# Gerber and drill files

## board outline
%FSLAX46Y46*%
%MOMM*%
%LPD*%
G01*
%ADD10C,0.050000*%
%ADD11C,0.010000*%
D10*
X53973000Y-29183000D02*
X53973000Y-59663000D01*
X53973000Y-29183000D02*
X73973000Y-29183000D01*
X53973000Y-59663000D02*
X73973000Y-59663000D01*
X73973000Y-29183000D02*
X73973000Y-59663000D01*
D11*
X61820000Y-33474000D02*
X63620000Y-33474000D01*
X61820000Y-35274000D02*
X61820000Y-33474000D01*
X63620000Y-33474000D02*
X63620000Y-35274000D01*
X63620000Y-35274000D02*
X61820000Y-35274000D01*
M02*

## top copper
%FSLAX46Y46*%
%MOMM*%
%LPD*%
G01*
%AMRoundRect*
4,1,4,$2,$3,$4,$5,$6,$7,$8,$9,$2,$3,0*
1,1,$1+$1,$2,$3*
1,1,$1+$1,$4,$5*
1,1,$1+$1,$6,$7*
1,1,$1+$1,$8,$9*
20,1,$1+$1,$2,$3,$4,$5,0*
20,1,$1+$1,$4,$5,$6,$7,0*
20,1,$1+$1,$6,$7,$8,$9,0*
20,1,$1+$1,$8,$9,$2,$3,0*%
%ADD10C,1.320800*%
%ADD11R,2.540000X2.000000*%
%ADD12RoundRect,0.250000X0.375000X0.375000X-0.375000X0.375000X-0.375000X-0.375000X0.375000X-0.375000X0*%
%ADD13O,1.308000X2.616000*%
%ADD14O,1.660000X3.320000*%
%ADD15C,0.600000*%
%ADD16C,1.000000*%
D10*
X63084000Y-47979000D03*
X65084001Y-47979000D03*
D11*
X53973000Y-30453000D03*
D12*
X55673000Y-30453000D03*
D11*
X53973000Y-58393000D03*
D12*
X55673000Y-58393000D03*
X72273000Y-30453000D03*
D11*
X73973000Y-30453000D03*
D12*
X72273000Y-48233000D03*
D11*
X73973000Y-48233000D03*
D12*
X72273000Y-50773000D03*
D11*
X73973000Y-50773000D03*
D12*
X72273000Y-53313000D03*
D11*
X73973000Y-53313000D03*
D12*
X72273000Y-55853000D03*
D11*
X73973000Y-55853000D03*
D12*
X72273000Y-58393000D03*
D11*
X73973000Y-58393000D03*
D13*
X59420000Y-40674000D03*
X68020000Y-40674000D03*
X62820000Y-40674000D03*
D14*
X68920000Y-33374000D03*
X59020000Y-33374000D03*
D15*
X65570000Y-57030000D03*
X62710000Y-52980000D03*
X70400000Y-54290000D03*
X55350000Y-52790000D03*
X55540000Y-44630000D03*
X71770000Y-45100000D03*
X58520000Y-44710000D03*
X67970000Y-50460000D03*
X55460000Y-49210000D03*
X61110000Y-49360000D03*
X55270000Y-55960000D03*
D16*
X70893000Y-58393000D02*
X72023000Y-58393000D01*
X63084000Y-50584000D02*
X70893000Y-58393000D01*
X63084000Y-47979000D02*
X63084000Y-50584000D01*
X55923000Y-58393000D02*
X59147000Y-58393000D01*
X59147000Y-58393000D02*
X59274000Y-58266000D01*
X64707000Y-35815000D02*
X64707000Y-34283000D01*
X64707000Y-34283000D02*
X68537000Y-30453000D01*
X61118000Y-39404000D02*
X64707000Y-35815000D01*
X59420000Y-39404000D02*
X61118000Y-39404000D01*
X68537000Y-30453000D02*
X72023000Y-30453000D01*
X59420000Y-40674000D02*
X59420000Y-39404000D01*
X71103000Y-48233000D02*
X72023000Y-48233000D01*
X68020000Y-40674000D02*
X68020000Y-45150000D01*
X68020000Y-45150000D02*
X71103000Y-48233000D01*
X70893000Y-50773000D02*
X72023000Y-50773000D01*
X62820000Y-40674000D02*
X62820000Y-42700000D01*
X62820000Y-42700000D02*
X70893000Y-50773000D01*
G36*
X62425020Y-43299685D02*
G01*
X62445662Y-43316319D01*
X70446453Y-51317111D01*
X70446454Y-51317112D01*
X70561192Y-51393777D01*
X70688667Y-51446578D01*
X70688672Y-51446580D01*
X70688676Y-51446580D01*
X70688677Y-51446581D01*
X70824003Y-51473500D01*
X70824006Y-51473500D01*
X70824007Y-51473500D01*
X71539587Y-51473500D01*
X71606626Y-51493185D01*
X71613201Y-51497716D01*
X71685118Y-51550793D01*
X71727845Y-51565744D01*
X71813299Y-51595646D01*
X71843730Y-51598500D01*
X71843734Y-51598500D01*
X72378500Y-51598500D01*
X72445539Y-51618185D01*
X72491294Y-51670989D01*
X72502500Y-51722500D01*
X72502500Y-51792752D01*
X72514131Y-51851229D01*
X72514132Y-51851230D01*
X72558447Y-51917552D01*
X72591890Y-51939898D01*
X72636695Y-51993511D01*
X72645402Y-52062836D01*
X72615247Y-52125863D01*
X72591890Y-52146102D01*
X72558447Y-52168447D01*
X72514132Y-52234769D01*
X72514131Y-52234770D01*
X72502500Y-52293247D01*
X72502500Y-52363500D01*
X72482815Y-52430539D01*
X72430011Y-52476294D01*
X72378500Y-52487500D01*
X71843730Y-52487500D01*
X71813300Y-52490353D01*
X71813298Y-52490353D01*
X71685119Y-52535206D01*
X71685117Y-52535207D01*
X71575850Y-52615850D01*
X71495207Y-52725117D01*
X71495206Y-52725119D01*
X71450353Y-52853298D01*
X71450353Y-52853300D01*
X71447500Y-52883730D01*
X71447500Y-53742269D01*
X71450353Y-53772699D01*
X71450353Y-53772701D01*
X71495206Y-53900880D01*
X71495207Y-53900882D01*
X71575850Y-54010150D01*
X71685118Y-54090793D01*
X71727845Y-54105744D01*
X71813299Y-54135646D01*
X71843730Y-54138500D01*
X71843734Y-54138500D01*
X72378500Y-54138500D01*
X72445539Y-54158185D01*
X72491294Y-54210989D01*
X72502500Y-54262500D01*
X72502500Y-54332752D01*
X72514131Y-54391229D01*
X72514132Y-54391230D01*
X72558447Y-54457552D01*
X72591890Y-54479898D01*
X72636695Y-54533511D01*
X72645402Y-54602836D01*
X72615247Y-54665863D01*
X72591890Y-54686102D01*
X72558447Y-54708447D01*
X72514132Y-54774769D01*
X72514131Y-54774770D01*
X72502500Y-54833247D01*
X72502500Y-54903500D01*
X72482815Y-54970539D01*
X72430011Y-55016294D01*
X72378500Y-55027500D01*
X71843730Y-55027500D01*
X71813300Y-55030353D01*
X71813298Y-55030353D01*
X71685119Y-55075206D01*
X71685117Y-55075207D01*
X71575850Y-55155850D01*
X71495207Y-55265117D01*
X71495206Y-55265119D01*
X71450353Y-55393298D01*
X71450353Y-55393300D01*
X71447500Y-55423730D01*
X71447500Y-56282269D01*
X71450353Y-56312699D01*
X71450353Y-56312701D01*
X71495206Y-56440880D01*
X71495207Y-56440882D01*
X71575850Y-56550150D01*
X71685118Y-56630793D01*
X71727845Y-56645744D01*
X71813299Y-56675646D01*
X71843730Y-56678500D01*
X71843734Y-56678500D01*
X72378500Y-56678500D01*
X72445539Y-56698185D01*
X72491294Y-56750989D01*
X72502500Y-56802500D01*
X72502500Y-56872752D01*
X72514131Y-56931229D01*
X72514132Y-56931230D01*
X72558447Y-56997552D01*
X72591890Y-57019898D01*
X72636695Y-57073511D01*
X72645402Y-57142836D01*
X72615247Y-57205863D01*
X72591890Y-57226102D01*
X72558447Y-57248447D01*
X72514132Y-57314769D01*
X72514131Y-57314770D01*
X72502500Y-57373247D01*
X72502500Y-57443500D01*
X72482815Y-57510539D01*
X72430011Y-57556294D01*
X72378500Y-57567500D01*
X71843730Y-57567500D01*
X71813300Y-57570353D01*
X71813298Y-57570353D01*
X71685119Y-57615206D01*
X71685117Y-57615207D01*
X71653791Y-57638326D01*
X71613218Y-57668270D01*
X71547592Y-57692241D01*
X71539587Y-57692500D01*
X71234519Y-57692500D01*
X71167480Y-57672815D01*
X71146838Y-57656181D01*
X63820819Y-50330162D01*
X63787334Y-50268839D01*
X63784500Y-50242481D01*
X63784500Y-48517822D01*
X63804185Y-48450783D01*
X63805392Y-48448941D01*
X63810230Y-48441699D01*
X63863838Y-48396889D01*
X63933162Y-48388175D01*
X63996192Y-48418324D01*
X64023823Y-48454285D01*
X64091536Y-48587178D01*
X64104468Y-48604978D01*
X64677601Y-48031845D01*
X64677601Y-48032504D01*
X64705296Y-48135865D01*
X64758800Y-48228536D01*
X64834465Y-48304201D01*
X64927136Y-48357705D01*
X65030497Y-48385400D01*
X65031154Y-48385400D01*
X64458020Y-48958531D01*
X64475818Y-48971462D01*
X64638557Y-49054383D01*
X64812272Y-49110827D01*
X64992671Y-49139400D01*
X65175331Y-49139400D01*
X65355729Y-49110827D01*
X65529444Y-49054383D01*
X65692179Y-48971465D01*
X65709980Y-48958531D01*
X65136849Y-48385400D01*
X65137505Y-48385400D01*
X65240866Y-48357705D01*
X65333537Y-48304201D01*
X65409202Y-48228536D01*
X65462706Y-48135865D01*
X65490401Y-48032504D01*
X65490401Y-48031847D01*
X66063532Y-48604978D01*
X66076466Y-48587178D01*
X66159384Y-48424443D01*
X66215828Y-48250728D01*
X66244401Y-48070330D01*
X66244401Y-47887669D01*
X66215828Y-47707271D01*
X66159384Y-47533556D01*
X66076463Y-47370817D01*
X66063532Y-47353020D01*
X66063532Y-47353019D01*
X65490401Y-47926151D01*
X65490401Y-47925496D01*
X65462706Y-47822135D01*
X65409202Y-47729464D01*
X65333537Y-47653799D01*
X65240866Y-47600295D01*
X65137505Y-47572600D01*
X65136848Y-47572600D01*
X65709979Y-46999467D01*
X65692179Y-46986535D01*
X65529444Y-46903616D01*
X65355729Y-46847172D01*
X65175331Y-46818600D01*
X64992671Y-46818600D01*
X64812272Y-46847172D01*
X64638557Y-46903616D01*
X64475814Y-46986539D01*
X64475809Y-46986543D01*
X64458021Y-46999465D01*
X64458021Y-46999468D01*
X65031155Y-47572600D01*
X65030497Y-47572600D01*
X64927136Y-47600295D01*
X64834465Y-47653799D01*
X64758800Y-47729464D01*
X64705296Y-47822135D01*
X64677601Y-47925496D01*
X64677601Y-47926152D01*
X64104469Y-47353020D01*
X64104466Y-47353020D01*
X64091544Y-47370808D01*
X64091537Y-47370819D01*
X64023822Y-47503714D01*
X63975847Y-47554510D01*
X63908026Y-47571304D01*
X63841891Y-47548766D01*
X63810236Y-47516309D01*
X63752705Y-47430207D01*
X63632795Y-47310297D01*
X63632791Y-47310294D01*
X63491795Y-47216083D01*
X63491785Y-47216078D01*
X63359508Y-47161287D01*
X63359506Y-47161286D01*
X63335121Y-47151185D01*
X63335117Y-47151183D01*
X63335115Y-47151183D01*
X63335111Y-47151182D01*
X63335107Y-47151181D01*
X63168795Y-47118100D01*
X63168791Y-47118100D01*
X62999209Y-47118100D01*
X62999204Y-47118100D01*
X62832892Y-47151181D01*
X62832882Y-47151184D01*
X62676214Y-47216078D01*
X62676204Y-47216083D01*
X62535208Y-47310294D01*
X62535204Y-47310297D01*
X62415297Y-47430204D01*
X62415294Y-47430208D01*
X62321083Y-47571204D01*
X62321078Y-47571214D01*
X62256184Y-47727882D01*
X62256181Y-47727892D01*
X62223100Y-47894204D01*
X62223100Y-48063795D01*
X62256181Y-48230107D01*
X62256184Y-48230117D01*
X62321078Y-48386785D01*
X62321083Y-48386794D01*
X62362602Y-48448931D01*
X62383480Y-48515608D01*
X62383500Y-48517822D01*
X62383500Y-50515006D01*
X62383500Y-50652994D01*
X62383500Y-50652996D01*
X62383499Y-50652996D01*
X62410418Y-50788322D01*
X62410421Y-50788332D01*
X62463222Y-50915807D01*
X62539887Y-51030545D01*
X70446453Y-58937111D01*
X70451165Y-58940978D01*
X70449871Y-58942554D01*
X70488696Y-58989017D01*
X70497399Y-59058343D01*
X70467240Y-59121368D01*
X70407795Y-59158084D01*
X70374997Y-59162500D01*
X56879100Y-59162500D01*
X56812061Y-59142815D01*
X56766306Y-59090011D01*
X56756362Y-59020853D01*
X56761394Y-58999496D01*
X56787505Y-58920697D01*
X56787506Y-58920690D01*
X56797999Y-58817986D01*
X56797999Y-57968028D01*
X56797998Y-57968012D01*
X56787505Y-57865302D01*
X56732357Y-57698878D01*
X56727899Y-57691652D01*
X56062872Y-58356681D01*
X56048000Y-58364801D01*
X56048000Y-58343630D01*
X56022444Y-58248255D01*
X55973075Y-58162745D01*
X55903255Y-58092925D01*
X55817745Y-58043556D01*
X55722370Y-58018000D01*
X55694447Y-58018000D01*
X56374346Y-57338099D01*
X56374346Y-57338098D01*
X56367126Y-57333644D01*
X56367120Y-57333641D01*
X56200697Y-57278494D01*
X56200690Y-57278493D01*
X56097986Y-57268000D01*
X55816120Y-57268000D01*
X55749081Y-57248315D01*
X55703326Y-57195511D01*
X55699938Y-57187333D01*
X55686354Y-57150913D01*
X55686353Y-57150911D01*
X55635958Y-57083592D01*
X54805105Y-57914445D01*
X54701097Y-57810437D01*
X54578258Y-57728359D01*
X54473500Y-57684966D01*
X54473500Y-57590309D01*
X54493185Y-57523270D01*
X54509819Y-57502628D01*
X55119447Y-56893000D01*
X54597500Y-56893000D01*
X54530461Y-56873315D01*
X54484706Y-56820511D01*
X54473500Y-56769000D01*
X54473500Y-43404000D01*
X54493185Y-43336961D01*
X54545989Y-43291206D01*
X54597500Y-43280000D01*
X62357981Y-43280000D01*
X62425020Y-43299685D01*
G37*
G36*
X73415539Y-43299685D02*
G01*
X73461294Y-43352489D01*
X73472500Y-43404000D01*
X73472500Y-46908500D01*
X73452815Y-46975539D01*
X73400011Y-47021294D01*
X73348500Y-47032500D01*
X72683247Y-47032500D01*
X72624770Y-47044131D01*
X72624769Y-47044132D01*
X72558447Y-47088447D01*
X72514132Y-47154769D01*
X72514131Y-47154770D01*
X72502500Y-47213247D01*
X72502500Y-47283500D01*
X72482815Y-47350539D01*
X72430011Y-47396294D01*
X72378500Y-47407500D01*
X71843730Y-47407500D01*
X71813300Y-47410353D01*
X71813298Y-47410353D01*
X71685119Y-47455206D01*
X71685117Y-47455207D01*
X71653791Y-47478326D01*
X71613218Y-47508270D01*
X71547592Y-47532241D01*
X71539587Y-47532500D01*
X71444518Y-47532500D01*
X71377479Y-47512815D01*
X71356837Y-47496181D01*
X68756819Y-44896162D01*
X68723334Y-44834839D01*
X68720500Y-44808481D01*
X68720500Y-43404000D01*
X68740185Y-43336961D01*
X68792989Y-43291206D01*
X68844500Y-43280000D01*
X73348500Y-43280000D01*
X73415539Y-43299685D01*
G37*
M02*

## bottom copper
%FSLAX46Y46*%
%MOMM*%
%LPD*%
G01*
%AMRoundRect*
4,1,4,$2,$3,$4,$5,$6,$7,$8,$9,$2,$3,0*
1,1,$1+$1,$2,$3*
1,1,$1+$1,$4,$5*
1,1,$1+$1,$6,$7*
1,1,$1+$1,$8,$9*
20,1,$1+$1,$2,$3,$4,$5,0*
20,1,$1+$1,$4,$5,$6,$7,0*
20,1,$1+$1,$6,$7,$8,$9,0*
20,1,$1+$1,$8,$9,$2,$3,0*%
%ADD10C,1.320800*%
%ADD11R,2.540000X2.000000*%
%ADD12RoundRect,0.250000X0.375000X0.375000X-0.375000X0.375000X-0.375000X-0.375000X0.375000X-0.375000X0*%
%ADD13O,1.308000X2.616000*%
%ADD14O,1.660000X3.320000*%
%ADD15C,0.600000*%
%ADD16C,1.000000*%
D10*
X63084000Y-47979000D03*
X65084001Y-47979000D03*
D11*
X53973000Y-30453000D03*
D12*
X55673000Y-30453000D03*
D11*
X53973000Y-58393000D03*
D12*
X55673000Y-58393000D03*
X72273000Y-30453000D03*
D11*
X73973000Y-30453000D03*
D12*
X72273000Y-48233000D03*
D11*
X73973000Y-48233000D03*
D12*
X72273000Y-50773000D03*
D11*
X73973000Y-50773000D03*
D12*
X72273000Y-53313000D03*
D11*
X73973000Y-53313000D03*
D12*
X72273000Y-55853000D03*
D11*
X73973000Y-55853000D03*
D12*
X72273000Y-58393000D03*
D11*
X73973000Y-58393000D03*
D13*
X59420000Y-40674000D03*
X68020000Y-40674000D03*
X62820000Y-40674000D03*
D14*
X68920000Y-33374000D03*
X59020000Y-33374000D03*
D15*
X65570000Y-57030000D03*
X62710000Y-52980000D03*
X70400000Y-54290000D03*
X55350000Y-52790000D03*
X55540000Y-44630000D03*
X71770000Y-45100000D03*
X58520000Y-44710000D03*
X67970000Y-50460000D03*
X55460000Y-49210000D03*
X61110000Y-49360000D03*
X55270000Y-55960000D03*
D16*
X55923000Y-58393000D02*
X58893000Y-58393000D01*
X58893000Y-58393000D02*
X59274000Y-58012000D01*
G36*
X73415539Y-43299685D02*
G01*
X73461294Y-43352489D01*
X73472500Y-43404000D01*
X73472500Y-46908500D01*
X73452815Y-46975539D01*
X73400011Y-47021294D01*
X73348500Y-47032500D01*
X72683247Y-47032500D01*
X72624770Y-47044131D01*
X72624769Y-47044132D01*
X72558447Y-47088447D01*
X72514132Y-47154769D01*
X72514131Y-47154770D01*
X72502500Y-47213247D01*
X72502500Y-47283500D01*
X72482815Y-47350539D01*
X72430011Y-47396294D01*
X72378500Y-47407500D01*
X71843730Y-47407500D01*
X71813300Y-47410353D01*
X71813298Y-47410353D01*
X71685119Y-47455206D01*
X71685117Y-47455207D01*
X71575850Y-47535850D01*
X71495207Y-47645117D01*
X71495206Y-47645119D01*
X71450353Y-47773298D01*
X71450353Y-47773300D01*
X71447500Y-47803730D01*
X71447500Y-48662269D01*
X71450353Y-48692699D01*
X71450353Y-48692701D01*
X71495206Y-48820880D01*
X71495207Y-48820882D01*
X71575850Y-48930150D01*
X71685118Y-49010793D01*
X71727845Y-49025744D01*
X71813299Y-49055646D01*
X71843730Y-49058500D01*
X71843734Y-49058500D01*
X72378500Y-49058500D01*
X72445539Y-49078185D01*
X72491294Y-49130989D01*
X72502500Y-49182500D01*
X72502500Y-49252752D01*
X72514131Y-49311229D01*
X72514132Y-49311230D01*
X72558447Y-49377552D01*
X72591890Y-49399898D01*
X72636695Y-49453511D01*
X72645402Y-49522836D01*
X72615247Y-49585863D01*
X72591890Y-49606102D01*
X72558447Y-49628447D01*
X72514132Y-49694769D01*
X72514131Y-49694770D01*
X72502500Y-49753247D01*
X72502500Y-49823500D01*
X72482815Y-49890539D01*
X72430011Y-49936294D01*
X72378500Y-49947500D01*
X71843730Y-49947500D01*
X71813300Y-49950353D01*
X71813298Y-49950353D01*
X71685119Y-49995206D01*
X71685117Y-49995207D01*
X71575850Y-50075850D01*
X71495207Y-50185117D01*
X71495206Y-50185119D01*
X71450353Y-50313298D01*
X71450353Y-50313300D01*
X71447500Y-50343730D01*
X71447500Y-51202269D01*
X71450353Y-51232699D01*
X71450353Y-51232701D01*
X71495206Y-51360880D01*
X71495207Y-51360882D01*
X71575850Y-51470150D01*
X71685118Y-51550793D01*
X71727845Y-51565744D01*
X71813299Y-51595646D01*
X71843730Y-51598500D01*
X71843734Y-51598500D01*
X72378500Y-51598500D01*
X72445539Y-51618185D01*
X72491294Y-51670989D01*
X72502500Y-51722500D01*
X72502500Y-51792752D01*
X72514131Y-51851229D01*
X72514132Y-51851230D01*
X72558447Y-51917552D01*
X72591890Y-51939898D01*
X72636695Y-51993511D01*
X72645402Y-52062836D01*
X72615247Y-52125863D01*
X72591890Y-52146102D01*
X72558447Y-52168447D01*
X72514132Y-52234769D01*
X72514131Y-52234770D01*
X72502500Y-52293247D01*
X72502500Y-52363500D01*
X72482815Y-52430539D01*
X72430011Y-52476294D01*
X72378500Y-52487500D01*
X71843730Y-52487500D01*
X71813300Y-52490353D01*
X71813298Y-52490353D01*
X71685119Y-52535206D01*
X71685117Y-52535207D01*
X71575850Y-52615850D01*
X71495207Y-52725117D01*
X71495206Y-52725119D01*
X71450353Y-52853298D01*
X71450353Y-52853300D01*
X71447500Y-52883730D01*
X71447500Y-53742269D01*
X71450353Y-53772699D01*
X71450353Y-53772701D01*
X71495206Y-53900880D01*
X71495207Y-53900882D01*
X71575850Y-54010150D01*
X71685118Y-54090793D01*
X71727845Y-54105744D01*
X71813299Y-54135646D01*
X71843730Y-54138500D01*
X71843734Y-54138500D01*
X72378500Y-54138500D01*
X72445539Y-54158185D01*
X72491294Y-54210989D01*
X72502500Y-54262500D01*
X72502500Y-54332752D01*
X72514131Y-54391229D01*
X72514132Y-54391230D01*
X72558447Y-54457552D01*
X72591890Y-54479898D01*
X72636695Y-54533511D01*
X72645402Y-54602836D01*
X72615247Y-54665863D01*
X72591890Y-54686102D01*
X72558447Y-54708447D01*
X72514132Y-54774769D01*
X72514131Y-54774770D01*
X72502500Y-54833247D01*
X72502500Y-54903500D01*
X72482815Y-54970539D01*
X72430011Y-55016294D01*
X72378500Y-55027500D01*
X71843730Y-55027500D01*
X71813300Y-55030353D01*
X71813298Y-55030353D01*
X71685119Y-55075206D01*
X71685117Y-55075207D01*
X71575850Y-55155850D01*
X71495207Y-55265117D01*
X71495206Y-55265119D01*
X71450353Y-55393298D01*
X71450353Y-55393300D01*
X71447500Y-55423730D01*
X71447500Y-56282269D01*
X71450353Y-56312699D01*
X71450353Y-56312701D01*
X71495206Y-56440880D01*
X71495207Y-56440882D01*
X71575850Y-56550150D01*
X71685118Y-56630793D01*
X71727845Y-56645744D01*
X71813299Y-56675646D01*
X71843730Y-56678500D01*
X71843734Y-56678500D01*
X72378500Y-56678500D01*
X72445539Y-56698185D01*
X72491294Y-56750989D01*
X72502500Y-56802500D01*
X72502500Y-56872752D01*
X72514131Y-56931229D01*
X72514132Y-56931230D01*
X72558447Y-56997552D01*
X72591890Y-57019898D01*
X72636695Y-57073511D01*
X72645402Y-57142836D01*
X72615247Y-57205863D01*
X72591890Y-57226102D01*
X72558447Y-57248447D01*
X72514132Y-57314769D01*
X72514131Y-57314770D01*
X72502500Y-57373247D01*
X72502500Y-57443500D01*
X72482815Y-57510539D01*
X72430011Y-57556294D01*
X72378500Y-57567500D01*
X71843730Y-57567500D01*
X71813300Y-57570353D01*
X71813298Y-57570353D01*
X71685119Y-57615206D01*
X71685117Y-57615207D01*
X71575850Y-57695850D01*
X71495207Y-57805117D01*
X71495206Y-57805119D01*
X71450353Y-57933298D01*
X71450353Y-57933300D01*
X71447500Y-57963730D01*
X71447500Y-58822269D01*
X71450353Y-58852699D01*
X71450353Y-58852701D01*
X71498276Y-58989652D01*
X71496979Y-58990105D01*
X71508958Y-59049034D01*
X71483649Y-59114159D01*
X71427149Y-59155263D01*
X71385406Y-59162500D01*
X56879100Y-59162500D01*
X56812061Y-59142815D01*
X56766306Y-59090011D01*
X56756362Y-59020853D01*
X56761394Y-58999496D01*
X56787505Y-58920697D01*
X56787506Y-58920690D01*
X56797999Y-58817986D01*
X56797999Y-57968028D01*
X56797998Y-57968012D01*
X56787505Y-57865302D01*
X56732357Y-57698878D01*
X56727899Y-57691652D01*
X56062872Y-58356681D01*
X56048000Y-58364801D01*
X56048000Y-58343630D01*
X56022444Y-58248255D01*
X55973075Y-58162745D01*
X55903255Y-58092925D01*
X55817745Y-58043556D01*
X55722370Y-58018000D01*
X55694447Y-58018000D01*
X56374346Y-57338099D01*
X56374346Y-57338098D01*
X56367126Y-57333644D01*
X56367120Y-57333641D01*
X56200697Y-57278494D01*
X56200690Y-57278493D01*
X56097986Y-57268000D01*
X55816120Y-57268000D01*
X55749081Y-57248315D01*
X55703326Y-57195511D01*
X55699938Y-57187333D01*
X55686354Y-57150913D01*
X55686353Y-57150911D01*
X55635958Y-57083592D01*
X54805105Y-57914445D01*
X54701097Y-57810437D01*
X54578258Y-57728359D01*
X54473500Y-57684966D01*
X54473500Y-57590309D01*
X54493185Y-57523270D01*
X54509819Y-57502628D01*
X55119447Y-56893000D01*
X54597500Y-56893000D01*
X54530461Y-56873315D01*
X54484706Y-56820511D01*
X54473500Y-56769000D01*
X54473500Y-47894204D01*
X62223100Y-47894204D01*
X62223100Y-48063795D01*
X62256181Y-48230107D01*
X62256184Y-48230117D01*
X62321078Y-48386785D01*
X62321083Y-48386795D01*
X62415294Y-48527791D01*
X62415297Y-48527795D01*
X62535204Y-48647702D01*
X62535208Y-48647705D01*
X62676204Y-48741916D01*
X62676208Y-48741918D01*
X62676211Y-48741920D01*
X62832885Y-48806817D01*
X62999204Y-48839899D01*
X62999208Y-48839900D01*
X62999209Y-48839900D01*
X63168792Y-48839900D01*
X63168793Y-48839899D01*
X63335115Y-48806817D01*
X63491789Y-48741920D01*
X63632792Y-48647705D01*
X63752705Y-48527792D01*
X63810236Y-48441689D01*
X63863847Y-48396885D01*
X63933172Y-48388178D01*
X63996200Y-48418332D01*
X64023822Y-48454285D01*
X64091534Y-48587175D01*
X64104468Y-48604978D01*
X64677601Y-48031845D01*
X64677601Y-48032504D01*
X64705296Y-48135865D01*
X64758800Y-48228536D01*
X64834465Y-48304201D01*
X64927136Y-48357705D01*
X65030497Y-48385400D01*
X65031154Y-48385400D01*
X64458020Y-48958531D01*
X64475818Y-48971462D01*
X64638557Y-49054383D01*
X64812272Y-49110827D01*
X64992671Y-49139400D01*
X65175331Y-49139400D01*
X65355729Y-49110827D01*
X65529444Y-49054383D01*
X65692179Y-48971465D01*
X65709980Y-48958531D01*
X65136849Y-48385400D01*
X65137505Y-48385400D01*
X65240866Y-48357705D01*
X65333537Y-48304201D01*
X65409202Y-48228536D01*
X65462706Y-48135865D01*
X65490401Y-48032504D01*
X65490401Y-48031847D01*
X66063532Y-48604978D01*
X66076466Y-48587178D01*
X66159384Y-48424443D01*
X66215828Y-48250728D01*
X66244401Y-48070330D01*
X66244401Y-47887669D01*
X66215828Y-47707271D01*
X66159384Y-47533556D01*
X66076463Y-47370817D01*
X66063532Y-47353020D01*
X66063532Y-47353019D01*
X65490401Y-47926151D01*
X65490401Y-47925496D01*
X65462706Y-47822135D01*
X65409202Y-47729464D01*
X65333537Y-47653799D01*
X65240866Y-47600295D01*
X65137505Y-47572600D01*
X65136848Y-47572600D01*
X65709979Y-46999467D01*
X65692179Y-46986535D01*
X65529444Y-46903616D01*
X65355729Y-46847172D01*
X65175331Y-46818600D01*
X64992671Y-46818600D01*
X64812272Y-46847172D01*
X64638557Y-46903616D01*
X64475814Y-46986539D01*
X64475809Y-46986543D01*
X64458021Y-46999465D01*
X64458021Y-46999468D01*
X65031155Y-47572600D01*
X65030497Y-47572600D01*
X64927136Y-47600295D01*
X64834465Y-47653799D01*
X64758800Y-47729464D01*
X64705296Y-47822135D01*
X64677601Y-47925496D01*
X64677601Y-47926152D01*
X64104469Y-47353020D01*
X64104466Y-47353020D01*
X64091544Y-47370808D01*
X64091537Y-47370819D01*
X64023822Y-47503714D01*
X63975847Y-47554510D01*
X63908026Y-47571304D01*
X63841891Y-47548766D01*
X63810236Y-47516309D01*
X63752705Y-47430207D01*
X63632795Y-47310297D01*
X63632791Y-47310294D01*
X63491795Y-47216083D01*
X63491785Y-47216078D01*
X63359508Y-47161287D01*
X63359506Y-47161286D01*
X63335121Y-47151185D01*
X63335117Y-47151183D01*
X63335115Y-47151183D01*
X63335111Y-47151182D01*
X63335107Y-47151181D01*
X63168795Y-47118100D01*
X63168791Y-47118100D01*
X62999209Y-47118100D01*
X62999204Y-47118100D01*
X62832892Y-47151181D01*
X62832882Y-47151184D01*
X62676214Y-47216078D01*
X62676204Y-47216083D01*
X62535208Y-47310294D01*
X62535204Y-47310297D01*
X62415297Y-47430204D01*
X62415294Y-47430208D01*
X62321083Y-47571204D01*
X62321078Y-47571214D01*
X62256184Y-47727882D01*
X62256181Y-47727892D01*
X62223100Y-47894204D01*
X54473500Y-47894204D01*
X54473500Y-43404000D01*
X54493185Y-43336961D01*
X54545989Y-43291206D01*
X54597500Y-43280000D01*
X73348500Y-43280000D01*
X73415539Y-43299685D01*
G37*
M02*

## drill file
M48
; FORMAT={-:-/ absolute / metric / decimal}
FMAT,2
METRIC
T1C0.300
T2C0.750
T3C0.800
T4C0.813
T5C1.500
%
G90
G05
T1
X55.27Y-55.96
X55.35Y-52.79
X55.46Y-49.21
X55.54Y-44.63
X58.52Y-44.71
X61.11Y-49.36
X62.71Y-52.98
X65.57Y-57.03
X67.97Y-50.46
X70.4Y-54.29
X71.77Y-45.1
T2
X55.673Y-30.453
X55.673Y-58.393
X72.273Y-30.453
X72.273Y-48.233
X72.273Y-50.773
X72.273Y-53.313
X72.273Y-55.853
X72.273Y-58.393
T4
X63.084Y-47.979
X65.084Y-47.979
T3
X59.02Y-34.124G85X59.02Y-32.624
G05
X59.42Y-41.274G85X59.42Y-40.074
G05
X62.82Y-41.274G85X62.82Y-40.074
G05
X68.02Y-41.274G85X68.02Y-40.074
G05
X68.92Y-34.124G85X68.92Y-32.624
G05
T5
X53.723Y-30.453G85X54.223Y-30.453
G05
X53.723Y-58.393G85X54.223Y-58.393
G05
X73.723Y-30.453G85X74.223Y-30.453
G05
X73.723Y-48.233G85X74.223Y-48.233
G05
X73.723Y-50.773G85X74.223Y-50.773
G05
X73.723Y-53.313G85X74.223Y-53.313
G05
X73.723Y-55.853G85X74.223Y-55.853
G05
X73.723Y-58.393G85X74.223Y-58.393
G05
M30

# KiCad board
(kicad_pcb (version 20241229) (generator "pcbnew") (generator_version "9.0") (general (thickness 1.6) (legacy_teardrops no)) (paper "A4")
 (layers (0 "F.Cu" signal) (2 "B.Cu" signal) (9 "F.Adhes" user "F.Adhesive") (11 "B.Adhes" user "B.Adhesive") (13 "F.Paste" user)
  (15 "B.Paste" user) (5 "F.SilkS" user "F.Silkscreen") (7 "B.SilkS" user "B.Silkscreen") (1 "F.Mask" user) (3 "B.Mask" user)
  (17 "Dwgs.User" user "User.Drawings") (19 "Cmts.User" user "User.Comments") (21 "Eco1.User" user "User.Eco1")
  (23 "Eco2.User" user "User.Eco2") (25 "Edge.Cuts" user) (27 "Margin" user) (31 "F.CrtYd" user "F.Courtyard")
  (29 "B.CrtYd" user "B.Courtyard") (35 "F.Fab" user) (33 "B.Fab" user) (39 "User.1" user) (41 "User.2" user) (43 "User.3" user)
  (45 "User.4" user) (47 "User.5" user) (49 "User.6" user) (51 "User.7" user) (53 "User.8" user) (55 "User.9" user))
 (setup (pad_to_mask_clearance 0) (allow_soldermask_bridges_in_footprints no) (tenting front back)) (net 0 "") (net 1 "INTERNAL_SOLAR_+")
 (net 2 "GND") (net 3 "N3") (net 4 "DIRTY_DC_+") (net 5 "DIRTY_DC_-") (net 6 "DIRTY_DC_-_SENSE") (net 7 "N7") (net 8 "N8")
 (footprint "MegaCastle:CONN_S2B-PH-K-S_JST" (layer "F.Cu") (at 63.084 47.979)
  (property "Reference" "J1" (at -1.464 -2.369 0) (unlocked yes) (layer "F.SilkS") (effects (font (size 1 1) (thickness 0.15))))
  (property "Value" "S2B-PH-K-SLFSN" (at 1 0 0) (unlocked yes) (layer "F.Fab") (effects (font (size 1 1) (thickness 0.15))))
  (pad "1" thru_hole circle (at 0 0) (size 1.3208 1.3208) (drill 0.8128) (layers "*.Cu" "*.Mask") (remove_unused_layers no)
   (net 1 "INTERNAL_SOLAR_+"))
  (pad "2" thru_hole circle (at 2.000001 0) (size 1.3208 1.3208) (drill 0.8128) (layers "*.Cu" "*.Mask") (remove_unused_layers no)
   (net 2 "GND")))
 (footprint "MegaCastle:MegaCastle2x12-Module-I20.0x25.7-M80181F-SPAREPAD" (layer "F.Cu") (at 63.973 44.423)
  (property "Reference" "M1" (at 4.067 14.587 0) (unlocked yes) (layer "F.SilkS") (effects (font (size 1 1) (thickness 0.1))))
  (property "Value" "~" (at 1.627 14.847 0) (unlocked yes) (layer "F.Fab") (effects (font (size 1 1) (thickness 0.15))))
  (fp_line (start -10 -15.24) (end -10 15.24) (stroke (width 0.05) (type default)) (layer "Edge.Cuts"))
  (fp_line (start -10 -15.24) (end 10 -15.24) (stroke (width 0.05) (type default)) (layer "Edge.Cuts"))
  (fp_line (start -10 15.24) (end 10 15.24) (stroke (width 0.05) (type default)) (layer "Edge.Cuts"))
  (fp_line (start 10 -15.24) (end 10 15.24) (stroke (width 0.05) (type default)) (layer "Edge.Cuts"))
  (pad "1" thru_hole rect (at -10 -13.97) (size 2.54 2) (drill oval 2 1.5) (layers "*.Cu" "*.Mask") (remove_unused_layers no) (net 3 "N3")
   (thermal_bridge_angle 45))
  (pad "1" thru_hole roundrect (at -8.3 -13.97 180) (size 1.25 1.25) (drill 0.75) (layers "*.Cu" "*.Mask") (remove_unused_layers no)
   (roundrect_rratio 0.2) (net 3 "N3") (thermal_bridge_angle 45))
  (pad "12" thru_hole rect (at -10 13.97) (size 2.54 2) (drill oval 2 1.5) (layers "*.Cu" "*.Mask") (remove_unused_layers no) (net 2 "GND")
   (thermal_bridge_angle 45))
  (pad "12" thru_hole roundrect (at -8.3 13.97 180) (size 1.25 1.25) (drill 0.75) (layers "*.Cu" "*.Mask") (remove_unused_layers no)
   (roundrect_rratio 0.2) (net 2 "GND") (thermal_bridge_angle 45))
  (pad "13" thru_hole roundrect (at 8.3 -13.97 180) (size 1.25 1.25) (drill 0.75) (layers "*.Cu" "*.Mask") (remove_unused_layers no)
   (roundrect_rratio 0.2) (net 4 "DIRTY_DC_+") (thermal_bridge_angle 45))
  (pad "13" thru_hole rect (at 10 -13.97) (size 2.54 2) (drill oval 2 1.5) (layers "*.Cu" "*.Mask") (remove_unused_layers no)
   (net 4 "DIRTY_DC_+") (thermal_bridge_angle 45))
  (pad "20" thru_hole roundrect (at 8.3 3.81 180) (size 1.25 1.25) (drill 0.75) (layers "*.Cu" "*.Mask") (remove_unused_layers no)
   (roundrect_rratio 0.2) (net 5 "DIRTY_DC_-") (thermal_bridge_angle 45))
  (pad "20" thru_hole rect (at 10 3.81) (size 2.54 2) (drill oval 2 1.5) (layers "*.Cu" "*.Mask") (remove_unused_layers no)
   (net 5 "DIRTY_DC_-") (thermal_bridge_angle 45))
  (pad "21" thru_hole roundrect (at 8.3 6.35 180) (size 1.25 1.25) (drill 0.75) (layers "*.Cu" "*.Mask") (remove_unused_layers no)
   (roundrect_rratio 0.2) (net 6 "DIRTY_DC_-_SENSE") (thermal_bridge_angle 45))
  (pad "21" thru_hole rect (at 10 6.35) (size 2.54 2) (drill oval 2 1.5) (layers "*.Cu" "*.Mask") (remove_unused_layers no)
   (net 6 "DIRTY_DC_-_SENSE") (thermal_bridge_angle 45))
  (pad "22" thru_hole roundrect (at 8.3 8.89 180) (size 1.25 1.25) (drill 0.75) (layers "*.Cu" "*.Mask") (remove_unused_layers no)
   (roundrect_rratio 0.2) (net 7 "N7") (thermal_bridge_angle 45))
  (pad "22" thru_hole rect (at 10 8.89) (size 2.54 2) (drill oval 2 1.5) (layers "*.Cu" "*.Mask") (remove_unused_layers no) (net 7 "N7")
   (thermal_bridge_angle 45))
  (pad "23" thru_hole roundrect (at 8.3 11.43 180) (size 1.25 1.25) (drill 0.75) (layers "*.Cu" "*.Mask") (remove_unused_layers no)
   (roundrect_rratio 0.2) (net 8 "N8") (thermal_bridge_angle 45))
  (pad "23" thru_hole rect (at 10 11.43) (size 2.54 2) (drill oval 2 1.5) (layers "*.Cu" "*.Mask") (remove_unused_layers no) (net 8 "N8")
   (thermal_bridge_angle 45))
  (pad "24" thru_hole roundrect (at 8.3 13.97 180) (size 1.25 1.25) (drill 0.75) (layers "*.Cu" "*.Mask") (remove_unused_layers no)
   (roundrect_rratio 0.2) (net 1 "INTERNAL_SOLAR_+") (thermal_bridge_angle 45))
  (pad "24" thru_hole rect (at 10 13.97) (size 2.54 2) (drill oval 2 1.5) (layers "*.Cu" "*.Mask") (remove_unused_layers no)
   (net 1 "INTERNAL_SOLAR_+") (thermal_bridge_angle 45))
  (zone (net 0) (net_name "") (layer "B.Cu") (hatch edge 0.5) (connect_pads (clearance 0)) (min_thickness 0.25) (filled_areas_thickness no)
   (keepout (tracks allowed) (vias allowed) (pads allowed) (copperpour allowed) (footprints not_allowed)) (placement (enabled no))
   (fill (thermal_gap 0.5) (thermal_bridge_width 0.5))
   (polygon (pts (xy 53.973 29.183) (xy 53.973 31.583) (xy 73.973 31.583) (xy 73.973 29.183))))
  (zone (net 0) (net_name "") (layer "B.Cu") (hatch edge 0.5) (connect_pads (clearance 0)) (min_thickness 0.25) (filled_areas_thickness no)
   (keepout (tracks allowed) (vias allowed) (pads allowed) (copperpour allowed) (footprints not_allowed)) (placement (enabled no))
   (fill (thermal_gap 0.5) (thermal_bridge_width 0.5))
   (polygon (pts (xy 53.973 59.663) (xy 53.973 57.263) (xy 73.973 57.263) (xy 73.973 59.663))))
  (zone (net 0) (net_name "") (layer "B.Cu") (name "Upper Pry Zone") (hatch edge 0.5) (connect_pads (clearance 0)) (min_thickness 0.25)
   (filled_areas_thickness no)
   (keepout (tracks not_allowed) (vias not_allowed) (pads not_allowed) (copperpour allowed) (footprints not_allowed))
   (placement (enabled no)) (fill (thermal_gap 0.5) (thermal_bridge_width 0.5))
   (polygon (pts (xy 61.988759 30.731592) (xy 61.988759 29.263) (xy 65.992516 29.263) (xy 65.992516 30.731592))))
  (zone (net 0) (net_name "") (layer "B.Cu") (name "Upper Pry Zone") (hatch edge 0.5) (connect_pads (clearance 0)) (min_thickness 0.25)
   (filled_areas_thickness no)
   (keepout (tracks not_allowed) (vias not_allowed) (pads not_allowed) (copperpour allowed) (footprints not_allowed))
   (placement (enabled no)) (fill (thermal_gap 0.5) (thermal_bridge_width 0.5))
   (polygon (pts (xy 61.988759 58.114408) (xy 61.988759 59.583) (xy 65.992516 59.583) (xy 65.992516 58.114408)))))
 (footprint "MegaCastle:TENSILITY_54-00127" (layer "F.Cu") (at 63.97 33.374 180)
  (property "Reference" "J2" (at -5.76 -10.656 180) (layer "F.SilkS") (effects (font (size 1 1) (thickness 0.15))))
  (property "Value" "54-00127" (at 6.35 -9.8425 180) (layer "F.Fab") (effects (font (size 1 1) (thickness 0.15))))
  (fp_line (start 2.15 -0.1) (end 0.35 -0.1) (stroke (width 0.01) (type solid)) (layer "Edge.Cuts"))
  (fp_line (start 2.15 -1.9) (end 2.15 -0.1) (stroke (width 0.01) (type solid)) (layer "Edge.Cuts"))
  (fp_line (start 0.35 -0.1) (end 0.35 -1.9) (stroke (width 0.01) (type solid)) (layer "Edge.Cuts"))
  (fp_line (start 0.35 -1.9) (end 2.15 -1.9) (stroke (width 0.01) (type solid)) (layer "Edge.Cuts"))
  (pad "A" thru_hole oval (at 4.55 -7.3 180) (size 1.308 2.616) (drill oval 0.8 2) (layers "*.Cu" "*.Mask") (remove_unused_layers no)
   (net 4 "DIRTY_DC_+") (solder_mask_margin 0.102))
  (pad "B" thru_hole oval (at -4.05 -7.3 180) (size 1.308 2.616) (drill oval 0.8 2) (layers "*.Cu" "*.Mask") (remove_unused_layers no)
   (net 5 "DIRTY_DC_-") (solder_mask_margin 0.102))
  (pad "C" thru_hole oval (at 1.15 -7.3 180) (size 1.308 2.616) (drill oval 0.8 2) (layers "*.Cu" "*.Mask") (remove_unused_layers no)
   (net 6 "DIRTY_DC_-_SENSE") (solder_mask_margin 0.102))
  (pad "SH1" thru_hole oval (at -4.95 0 180) (size 1.66 3.32) (drill oval 0.8 2.3) (layers "*.Cu" "*.Mask") (remove_unused_layers no)
   (solder_mask_margin 0.102))
  (pad "SH2" thru_hole oval (at 4.95 0 180) (size 1.66 3.32) (drill oval 0.8 2.3) (layers "*.Cu" "*.Mask") (remove_unused_layers no)
   (solder_mask_margin 0.102)))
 (segment (start 70.893 58.393) (end 72.023 58.393) (width 1) (layer "F.Cu") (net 1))
 (segment (start 63.084 50.584) (end 70.893 58.393) (width 1) (layer "F.Cu") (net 1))
 (segment (start 63.084 47.979) (end 63.084 50.584) (width 1) (layer "F.Cu") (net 1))
 (segment (start 55.923 58.393) (end 59.147 58.393) (width 1) (layer "F.Cu") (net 2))
 (segment (start 59.147 58.393) (end 59.274 58.266) (width 1) (layer "F.Cu") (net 2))
 (via (at 65.57 57.03) (size 0.6) (drill 0.3) (layers "F.Cu" "B.Cu") (free yes) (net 2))
 (via (at 62.71 52.98) (size 0.6) (drill 0.3) (layers "F.Cu" "B.Cu") (free yes) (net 2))
 (via (at 70.4 54.29) (size 0.6) (drill 0.3) (layers "F.Cu" "B.Cu") (free yes) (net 2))
 (via (at 55.35 52.79) (size 0.6) (drill 0.3) (layers "F.Cu" "B.Cu") (free yes) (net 2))
 (via (at 55.54 44.63) (size 0.6) (drill 0.3) (layers "F.Cu" "B.Cu") (free yes) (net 2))
 (via (at 71.77 45.1) (size 0.6) (drill 0.3) (layers "F.Cu" "B.Cu") (free yes) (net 2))
 (via (at 58.52 44.71) (size 0.6) (drill 0.3) (layers "F.Cu" "B.Cu") (free yes) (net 2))
 (via (at 67.97 50.46) (size 0.6) (drill 0.3) (layers "F.Cu" "B.Cu") (free yes) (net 2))
 (via (at 55.46 49.21) (size 0.6) (drill 0.3) (layers "F.Cu" "B.Cu") (free yes) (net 2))
 (via (at 61.11 49.36) (size 0.6) (drill 0.3) (layers "F.Cu" "B.Cu") (free yes) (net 2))
 (via (at 55.27 55.96) (size 0.6) (drill 0.3) (layers "F.Cu" "B.Cu") (free yes) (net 2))
 (segment (start 55.923 58.393) (end 58.893 58.393) (width 1) (layer "B.Cu") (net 2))
 (segment (start 58.893 58.393) (end 59.274 58.012) (width 1) (layer "B.Cu") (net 2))
 (segment (start 64.707 35.815) (end 64.707 34.283) (width 1) (layer "F.Cu") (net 4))
 (segment (start 64.707 34.283) (end 68.537 30.453) (width 1) (layer "F.Cu") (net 4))
 (segment (start 61.118 39.404) (end 64.707 35.815) (width 1) (layer "F.Cu") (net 4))
 (segment (start 59.42 39.404) (end 61.118 39.404) (width 1) (layer "F.Cu") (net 4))
 (segment (start 68.537 30.453) (end 72.023 30.453) (width 1) (layer "F.Cu") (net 4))
 (segment (start 59.42 40.674) (end 59.42 39.404) (width 1) (layer "F.Cu") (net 4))
 (segment (start 71.103 48.233) (end 72.023 48.233) (width 1) (layer "F.Cu") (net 5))
 (segment (start 68.02 40.674) (end 68.02 45.15) (width 1) (layer "F.Cu") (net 5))
 (segment (start 68.02 45.15) (end 71.103 48.233) (width 1) (layer "F.Cu") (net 5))
 (segment (start 70.893 50.773) (end 72.023 50.773) (width 1) (layer "F.Cu") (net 6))
 (segment (start 62.82 40.674) (end 62.82 42.7) (width 1) (layer "F.Cu") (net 6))
 (segment (start 62.82 42.7) (end 70.893 50.773) (width 1) (layer "F.Cu") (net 6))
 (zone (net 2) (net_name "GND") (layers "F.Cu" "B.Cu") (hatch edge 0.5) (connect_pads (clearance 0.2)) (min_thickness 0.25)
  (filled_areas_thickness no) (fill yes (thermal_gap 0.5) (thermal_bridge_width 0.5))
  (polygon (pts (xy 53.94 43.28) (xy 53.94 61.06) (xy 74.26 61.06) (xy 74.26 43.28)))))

